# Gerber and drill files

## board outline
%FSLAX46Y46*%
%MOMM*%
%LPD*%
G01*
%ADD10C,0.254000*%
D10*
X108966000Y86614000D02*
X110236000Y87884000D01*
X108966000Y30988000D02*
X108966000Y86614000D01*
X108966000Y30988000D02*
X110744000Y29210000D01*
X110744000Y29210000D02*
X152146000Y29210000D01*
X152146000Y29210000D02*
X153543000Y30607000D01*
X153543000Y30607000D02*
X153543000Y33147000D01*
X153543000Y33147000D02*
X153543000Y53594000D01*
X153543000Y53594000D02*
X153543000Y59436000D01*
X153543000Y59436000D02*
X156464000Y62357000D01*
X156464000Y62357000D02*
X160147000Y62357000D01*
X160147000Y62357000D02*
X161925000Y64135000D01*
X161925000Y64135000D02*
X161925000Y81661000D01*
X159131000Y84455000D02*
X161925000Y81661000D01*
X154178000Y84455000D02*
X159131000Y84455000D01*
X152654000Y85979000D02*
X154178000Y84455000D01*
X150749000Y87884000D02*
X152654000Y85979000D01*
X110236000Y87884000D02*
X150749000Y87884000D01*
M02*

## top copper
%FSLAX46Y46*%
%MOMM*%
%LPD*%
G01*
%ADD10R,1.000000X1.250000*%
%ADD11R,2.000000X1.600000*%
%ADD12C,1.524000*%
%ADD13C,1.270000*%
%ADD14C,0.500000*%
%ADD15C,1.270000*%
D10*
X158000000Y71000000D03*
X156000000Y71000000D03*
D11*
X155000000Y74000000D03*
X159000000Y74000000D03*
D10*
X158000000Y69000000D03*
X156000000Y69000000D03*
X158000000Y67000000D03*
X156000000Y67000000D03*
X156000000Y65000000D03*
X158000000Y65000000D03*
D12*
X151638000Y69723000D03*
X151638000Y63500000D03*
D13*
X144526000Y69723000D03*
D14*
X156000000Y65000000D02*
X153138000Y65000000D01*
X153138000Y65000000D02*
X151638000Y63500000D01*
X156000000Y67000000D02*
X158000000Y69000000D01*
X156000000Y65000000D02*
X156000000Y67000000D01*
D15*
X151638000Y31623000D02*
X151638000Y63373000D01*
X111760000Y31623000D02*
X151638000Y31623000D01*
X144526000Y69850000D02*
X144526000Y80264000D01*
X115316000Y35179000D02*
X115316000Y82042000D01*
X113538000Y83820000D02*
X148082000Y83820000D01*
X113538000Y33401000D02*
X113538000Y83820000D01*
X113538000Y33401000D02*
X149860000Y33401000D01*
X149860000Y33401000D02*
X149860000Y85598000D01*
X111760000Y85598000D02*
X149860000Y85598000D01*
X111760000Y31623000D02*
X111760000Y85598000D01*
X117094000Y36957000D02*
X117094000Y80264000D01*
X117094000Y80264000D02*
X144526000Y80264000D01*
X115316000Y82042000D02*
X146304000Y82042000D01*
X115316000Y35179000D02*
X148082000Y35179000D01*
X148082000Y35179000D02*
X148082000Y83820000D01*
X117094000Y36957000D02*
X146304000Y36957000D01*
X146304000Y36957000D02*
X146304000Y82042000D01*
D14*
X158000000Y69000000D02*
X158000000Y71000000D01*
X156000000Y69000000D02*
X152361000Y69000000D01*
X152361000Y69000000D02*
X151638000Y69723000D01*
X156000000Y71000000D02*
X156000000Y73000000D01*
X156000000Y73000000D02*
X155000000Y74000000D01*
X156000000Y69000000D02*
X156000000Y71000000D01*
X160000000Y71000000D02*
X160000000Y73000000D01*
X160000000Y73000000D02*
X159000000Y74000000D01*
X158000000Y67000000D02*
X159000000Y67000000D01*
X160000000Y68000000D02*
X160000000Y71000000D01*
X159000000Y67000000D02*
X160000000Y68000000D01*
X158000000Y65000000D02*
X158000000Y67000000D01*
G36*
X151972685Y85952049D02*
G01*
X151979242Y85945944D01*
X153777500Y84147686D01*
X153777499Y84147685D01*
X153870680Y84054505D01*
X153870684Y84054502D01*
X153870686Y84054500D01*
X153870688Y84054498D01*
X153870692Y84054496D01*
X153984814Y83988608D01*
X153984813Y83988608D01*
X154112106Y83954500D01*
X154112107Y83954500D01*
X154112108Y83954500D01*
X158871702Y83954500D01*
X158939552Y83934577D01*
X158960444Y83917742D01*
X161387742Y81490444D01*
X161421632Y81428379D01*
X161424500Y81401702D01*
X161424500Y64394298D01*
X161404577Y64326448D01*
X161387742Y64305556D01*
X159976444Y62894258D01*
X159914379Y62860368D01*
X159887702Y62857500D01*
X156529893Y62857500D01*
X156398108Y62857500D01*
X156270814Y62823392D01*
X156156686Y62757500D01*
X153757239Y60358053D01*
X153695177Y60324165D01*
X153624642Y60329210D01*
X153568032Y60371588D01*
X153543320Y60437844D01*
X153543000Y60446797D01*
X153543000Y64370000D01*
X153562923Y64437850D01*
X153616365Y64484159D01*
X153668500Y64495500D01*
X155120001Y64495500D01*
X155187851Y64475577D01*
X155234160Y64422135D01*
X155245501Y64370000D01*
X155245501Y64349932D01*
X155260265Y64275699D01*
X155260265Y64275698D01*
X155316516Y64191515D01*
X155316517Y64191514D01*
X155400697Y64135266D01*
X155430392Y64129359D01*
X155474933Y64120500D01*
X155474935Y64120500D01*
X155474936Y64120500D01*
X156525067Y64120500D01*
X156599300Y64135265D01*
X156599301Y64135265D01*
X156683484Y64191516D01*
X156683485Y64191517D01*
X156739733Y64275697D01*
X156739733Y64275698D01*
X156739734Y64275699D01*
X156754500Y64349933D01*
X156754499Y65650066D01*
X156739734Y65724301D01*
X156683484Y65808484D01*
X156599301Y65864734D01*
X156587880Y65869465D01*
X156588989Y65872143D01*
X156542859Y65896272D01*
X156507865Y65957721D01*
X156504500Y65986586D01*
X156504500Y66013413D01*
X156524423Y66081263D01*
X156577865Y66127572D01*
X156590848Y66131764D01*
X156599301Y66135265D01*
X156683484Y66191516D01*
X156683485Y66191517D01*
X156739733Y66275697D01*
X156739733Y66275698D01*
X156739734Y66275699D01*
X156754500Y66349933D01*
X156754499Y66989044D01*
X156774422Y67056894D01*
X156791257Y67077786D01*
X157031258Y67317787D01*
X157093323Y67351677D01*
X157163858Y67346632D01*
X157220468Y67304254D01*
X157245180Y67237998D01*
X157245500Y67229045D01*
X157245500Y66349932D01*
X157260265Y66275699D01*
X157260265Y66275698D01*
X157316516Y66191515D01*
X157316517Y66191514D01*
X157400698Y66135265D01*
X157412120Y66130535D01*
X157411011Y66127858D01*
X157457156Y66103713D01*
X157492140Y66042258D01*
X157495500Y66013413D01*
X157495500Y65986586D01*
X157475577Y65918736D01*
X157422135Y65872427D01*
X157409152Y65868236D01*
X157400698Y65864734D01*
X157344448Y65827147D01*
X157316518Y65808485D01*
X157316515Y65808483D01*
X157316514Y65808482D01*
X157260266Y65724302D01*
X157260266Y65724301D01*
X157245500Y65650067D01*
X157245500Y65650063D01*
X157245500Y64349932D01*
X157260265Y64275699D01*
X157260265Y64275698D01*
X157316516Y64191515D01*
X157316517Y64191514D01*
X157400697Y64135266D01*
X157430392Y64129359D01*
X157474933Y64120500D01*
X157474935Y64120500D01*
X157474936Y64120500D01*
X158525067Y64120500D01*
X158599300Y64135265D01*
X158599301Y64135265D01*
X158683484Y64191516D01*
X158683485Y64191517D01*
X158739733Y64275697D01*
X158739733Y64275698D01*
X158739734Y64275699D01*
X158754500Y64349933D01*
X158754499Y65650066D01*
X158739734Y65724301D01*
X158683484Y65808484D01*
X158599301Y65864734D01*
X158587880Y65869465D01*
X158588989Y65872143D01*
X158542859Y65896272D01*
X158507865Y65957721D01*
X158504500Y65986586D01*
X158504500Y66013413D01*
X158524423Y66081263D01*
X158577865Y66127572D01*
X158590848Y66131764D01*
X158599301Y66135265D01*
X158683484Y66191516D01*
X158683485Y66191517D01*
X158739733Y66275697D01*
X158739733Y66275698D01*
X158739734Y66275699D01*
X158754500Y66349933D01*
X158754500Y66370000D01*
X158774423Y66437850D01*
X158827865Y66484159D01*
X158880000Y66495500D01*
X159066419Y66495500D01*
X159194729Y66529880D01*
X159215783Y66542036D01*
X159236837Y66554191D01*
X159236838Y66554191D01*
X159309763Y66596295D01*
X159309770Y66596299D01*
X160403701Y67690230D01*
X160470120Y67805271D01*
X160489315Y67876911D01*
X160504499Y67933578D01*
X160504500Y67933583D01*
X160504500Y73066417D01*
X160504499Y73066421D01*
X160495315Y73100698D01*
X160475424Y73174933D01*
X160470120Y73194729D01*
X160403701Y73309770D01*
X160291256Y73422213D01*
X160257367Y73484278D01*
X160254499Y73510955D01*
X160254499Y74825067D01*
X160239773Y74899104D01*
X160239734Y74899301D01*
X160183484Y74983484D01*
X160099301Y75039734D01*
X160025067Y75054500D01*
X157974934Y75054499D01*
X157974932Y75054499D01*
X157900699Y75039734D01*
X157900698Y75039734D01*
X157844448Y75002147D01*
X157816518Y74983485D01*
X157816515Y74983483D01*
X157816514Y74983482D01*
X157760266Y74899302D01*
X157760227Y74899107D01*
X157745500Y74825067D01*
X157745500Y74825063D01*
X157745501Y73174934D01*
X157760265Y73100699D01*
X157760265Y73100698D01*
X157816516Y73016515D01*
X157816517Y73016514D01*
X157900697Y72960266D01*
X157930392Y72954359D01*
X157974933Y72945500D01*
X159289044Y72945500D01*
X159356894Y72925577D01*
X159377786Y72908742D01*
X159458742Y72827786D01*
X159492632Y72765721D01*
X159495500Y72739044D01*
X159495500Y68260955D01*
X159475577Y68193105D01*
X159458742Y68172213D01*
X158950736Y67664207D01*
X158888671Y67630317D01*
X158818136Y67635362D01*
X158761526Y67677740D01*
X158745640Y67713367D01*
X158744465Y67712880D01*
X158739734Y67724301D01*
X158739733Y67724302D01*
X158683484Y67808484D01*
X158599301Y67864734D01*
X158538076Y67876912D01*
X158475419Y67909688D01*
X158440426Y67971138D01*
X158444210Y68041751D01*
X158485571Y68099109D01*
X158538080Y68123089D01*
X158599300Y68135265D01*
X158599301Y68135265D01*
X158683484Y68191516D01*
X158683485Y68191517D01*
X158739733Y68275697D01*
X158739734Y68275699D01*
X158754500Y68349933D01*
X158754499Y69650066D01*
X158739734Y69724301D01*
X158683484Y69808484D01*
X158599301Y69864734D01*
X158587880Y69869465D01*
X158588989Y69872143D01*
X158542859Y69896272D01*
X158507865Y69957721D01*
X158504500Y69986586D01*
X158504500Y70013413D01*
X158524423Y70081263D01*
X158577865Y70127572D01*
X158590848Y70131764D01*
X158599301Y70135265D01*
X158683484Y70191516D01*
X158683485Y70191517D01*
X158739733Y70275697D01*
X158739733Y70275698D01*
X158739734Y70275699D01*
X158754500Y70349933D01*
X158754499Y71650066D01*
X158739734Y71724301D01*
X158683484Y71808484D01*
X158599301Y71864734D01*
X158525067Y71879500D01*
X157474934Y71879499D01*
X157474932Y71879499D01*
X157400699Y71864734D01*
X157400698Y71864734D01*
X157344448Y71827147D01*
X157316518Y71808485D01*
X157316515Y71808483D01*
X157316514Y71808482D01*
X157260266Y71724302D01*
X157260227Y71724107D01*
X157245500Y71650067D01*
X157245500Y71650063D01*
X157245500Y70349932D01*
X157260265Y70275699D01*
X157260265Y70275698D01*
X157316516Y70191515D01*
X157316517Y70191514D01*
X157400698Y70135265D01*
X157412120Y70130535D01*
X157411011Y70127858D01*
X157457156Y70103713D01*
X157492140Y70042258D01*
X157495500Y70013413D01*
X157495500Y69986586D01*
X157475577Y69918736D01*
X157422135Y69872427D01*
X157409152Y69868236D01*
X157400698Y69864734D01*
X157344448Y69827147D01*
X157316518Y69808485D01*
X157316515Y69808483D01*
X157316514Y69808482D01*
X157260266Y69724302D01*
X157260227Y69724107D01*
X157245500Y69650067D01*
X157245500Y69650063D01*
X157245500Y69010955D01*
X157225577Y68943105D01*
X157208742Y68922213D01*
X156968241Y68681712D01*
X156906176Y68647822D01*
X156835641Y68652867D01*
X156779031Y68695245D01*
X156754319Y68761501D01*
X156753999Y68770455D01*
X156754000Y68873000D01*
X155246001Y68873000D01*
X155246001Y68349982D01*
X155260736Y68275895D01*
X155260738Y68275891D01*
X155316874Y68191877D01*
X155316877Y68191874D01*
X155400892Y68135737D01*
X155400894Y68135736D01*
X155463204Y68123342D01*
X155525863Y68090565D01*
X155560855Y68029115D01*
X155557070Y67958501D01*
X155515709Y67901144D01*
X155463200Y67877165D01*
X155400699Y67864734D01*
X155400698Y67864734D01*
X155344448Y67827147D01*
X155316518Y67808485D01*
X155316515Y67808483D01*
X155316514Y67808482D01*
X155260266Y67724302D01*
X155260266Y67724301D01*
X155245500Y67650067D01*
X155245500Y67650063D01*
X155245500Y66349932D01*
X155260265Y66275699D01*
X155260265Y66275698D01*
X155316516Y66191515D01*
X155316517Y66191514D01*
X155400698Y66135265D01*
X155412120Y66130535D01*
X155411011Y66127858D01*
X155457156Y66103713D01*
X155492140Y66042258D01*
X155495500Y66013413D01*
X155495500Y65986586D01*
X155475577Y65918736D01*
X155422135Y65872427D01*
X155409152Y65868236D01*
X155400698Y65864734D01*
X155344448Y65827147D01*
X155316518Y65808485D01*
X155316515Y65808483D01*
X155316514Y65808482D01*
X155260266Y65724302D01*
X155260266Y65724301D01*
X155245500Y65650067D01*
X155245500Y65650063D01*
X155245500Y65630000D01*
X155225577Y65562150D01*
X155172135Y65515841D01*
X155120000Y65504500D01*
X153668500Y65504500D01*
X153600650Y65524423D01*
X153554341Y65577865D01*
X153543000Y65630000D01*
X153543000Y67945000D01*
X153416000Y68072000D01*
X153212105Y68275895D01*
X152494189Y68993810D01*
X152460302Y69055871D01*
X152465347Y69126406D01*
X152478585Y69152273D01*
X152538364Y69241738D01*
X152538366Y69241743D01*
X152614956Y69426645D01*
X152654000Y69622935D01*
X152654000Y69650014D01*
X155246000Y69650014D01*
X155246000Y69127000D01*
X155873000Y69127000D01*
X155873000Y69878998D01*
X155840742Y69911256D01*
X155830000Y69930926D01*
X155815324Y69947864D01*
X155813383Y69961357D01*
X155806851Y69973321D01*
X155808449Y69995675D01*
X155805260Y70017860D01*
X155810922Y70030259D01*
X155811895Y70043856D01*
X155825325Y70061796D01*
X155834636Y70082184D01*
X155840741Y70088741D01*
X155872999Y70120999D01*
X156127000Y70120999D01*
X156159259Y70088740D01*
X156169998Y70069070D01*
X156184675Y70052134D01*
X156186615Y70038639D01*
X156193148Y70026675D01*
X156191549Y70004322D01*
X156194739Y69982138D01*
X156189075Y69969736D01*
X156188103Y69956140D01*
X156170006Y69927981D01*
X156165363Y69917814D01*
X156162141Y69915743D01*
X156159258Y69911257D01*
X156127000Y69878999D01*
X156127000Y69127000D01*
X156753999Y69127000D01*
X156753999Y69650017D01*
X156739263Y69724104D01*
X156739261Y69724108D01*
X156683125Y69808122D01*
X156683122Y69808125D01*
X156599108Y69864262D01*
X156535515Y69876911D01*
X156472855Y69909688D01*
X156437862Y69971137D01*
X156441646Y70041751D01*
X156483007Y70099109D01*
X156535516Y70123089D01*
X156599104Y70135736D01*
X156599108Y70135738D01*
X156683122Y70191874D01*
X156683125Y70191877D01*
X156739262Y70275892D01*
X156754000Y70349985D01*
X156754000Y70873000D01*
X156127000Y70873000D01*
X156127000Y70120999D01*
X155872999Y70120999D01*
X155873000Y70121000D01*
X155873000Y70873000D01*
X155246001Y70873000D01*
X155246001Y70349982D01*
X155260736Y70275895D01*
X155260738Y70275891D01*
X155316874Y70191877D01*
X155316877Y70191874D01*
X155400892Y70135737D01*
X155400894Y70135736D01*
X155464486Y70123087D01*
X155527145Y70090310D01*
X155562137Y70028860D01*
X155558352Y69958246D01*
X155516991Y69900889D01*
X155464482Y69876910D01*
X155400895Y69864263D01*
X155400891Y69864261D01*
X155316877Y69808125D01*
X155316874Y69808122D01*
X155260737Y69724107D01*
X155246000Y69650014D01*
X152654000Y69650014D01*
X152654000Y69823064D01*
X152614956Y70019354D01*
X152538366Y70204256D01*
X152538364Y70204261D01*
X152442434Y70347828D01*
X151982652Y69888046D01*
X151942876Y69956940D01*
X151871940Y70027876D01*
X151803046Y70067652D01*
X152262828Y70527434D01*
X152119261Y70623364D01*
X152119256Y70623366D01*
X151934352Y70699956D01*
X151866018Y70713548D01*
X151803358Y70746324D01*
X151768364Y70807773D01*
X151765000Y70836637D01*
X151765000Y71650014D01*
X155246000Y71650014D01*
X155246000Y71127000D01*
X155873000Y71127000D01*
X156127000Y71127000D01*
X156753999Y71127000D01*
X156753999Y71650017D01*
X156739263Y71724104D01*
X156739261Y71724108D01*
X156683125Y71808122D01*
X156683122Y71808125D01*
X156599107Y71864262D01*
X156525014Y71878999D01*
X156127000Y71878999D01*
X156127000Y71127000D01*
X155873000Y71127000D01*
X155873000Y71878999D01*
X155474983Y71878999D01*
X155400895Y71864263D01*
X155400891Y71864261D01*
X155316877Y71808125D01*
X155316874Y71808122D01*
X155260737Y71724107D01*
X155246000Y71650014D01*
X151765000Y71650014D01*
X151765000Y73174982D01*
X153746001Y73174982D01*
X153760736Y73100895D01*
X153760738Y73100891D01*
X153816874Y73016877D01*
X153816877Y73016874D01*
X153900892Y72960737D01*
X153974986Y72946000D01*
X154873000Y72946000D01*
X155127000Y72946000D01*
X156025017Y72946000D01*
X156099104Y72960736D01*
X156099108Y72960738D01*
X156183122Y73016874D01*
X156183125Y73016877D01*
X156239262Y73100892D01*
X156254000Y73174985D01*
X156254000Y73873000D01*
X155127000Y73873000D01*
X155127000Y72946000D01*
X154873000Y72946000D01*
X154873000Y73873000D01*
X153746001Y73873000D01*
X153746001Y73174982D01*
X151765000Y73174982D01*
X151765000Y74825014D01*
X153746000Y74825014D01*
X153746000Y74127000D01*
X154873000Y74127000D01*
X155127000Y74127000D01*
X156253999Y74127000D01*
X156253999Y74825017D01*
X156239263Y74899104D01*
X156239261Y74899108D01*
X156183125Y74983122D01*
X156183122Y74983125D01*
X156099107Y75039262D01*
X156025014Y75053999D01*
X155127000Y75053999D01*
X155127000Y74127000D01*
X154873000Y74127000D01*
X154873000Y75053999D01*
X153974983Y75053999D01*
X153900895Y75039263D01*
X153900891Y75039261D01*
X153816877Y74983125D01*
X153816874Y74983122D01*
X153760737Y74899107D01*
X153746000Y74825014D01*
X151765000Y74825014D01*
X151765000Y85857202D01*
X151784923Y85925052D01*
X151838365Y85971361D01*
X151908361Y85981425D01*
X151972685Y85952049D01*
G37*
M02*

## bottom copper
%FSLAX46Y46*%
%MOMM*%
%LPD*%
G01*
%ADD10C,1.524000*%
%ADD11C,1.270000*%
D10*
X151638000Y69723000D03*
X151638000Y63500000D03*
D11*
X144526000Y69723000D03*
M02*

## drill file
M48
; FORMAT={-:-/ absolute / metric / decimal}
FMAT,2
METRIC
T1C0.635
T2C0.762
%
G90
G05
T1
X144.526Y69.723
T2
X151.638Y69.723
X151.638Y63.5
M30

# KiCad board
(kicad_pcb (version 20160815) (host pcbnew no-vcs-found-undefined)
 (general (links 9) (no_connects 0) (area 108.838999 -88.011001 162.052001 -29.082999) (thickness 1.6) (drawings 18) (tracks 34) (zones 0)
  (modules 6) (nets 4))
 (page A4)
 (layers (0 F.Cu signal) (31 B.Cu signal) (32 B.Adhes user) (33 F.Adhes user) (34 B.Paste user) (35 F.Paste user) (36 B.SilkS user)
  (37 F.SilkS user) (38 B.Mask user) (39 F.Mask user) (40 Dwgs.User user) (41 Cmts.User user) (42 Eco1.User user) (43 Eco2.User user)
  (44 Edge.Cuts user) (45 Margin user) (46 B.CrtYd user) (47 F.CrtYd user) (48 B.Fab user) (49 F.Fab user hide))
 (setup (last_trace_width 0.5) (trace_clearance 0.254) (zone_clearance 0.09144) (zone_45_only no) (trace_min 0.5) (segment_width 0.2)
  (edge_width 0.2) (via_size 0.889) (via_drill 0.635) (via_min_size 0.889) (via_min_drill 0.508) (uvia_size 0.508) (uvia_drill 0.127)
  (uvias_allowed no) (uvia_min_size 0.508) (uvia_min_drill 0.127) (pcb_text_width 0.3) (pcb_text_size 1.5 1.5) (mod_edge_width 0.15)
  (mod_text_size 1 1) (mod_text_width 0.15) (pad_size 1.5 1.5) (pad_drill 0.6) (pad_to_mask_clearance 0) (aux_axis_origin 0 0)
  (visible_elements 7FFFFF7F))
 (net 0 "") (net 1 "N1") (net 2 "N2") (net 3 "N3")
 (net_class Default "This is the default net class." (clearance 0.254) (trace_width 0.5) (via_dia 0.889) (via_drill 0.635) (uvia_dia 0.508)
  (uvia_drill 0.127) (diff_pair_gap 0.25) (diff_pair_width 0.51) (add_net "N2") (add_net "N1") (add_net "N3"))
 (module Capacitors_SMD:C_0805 (layer F.Cu) (at 157 -71)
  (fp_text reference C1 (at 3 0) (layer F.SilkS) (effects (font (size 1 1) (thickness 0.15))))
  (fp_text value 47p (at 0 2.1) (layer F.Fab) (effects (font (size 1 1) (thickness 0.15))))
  (pad 2 smd rect (at 1 0) (size 1 1.25) (layers F.Cu F.Paste F.Mask) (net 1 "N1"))
  (pad 1 smd rect (at -1 0) (size 1 1.25) (layers F.Cu F.Paste F.Mask) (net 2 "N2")))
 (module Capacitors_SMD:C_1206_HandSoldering (layer F.Cu) (at 157 -74 180)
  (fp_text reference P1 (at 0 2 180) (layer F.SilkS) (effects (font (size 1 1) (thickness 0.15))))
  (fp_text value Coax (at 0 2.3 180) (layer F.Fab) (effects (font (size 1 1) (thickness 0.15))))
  (pad 2 smd rect (at 2 0 180) (size 2 1.6) (layers F.Cu F.Paste F.Mask) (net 2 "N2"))
  (pad 1 smd rect (at -2 0 180) (size 2 1.6) (layers F.Cu F.Paste F.Mask) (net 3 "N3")))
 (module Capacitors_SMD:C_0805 (layer F.Cu) (at 157 -69)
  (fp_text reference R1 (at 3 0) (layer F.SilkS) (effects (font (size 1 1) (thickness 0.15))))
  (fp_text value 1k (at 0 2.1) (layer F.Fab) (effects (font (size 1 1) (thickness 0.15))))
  (pad 2 smd rect (at 1 0) (size 1 1.25) (layers F.Cu F.Paste F.Mask) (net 1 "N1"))
  (pad 1 smd rect (at -1 0) (size 1 1.25) (layers F.Cu F.Paste F.Mask) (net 2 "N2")))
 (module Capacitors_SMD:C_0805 (layer F.Cu) (at 157 -67)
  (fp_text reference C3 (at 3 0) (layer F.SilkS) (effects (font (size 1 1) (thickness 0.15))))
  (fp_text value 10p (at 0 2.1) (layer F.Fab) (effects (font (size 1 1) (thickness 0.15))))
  (pad 2 smd rect (at 1 0) (size 1 1.25) (layers F.Cu F.Paste F.Mask) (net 3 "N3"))
  (pad 1 smd rect (at -1 0) (size 1 1.25) (layers F.Cu F.Paste F.Mask) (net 1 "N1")))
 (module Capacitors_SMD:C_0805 (layer F.Cu) (at 157 -65)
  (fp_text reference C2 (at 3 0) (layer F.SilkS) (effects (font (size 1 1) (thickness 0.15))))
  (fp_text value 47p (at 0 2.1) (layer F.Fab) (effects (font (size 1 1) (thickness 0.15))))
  (pad 1 smd rect (at -1 0) (size 1 1.25) (layers F.Cu F.Paste F.Mask) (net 1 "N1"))
  (pad 2 smd rect (at 1 0) (size 1 1.25) (layers F.Cu F.Paste F.Mask) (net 3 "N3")))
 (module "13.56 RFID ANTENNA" (layer F.Cu) (at 111.76 -31.623)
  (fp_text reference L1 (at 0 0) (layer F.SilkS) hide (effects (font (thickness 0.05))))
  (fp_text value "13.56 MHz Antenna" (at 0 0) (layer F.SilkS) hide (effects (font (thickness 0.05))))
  (pad 2 thru_hole circle (at 39.878 -38.1) (size 1.524 1.524) (drill 0.762) (layers *.Cu *.Paste *.Mask) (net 2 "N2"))
  (pad 1 thru_hole circle (at 39.878 -31.877) (size 1.524 1.524) (drill 0.762) (layers *.Cu *.Paste *.Mask) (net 1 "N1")))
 (gr_line (start 108.966 -86.614) (end 110.236 -87.884) (layer Edge.Cuts) (width 0.254))
 (gr_line (start 108.966 -30.988) (end 108.966 -86.614) (layer Edge.Cuts) (width 0.254))
 (gr_line (start 108.966 -30.988) (end 110.744 -29.21) (layer Edge.Cuts) (width 0.254))
 (gr_line (start 110.744 -29.21) (end 152.146 -29.21) (layer Edge.Cuts) (width 0.254))
 (gr_line (start 152.146 -29.21) (end 153.543 -30.607) (layer Edge.Cuts) (width 0.254))
 (gr_line (start 153.543 -30.607) (end 153.543 -33.147) (layer Edge.Cuts) (width 0.254))
 (gr_line (start 153.543 -33.147) (end 153.543 -53.594) (layer Edge.Cuts) (width 0.254))
 (gr_line (start 153.543 -53.594) (end 153.543 -59.436) (layer Edge.Cuts) (width 0.254))
 (gr_line (start 153.543 -59.436) (end 156.464 -62.357) (layer Edge.Cuts) (width 0.254))
 (gr_line (start 156.464 -62.357) (end 160.147 -62.357) (layer Edge.Cuts) (width 0.254))
 (gr_line (start 160.147 -62.357) (end 161.925 -64.135) (layer Edge.Cuts) (width 0.254))
 (gr_line (start 161.925 -64.135) (end 161.925 -81.661) (layer Edge.Cuts) (width 0.254))
 (gr_line (start 159.131 -84.455) (end 161.925 -81.661) (layer Edge.Cuts) (width 0.254))
 (gr_line (start 154.178 -84.455) (end 159.131 -84.455) (layer Edge.Cuts) (width 0.254))
 (gr_line (start 152.654 -85.979) (end 154.178 -84.455) (layer Edge.Cuts) (width 0.254))
 (gr_line (start 150.749 -87.884) (end 152.654 -85.979) (layer Edge.Cuts) (width 0.254))
 (gr_line (start 110.236 -87.884) (end 150.749 -87.884) (layer Edge.Cuts) (width 0.254))
 (segment (start 156 -65) (end 153.138 -65) (width 0.5) (layer F.Cu) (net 1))
 (segment (start 153.138 -65) (end 151.638 -63.5) (width 0.5) (layer F.Cu) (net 1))
 (segment (start 156 -67) (end 158 -69) (width 0.5) (layer F.Cu) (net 1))
 (segment (start 156 -65) (end 156 -67) (width 0.5) (layer F.Cu) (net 1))
 (via (at 144.526 -69.723) (size 1.27) (layers F.Cu B.Cu) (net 1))
 (segment (start 151.638 -31.623) (end 151.638 -63.373) (width 1.27) (layer F.Cu) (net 1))
 (segment (start 111.76 -31.623) (end 151.638 -31.623) (width 1.27) (layer F.Cu) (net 1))
 (segment (start 144.526 -69.85) (end 144.526 -80.264) (width 1.27) (layer F.Cu) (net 1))
 (segment (start 115.316 -35.179) (end 115.316 -82.042) (width 1.27) (layer F.Cu) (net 1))
 (segment (start 113.538 -83.82) (end 148.082 -83.82) (width 1.27) (layer F.Cu) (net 1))
 (segment (start 113.538 -33.401) (end 113.538 -83.82) (width 1.27) (layer F.Cu) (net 1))
 (segment (start 113.538 -33.401) (end 149.86 -33.401) (width 1.27) (layer F.Cu) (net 1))
 (segment (start 149.86 -33.401) (end 149.86 -85.598) (width 1.27) (layer F.Cu) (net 1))
 (segment (start 111.76 -85.598) (end 149.86 -85.598) (width 1.27) (layer F.Cu) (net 1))
 (segment (start 111.76 -31.623) (end 111.76 -85.598) (width 1.27) (layer F.Cu) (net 1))
 (segment (start 117.094 -36.957) (end 117.094 -80.264) (width 1.27) (layer F.Cu) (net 1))
 (segment (start 117.094 -80.264) (end 144.526 -80.264) (width 1.27) (layer F.Cu) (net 1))
 (segment (start 115.316 -82.042) (end 146.304 -82.042) (width 1.27) (layer F.Cu) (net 1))
 (segment (start 115.316 -35.179) (end 148.082 -35.179) (width 1.27) (layer F.Cu) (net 1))
 (segment (start 148.082 -35.179) (end 148.082 -83.82) (width 1.27) (layer F.Cu) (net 1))
 (segment (start 117.094 -36.957) (end 146.304 -36.957) (width 1.27) (layer F.Cu) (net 1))
 (segment (start 146.304 -36.957) (end 146.304 -82.042) (width 1.27) (layer F.Cu) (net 1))
 (segment (start 158 -69) (end 158 -71) (width 0.5) (layer F.Cu) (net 1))
 (segment (start 156 -69) (end 152.361 -69) (width 0.5) (layer F.Cu) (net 2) (status 400000))
 (segment (start 152.361 -69) (end 151.638 -69.723) (width 0.5) (layer F.Cu) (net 2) (status 800000))
 (segment (start 156 -71) (end 156 -73) (width 0.5) (layer F.Cu) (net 2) (status 400000))
 (segment (start 156 -73) (end 155 -74) (width 0.5) (layer F.Cu) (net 2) (status 800000))
 (segment (start 156 -69) (end 156 -71) (width 0.5) (layer F.Cu) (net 2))
 (segment (start 160 -71) (end 160 -73) (width 0.5) (layer F.Cu) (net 3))
 (segment (start 160 -73) (end 159 -74) (width 0.5) (layer F.Cu) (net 3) (status 800000))
 (segment (start 158 -67) (end 159 -67) (width 0.5) (layer F.Cu) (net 3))
 (segment (start 160 -68) (end 160 -71) (width 0.5) (layer F.Cu) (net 3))
 (segment (start 159 -67) (end 160 -68) (width 0.5) (layer F.Cu) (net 3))
 (segment (start 158 -65) (end 158 -67) (width 0.5) (layer F.Cu) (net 3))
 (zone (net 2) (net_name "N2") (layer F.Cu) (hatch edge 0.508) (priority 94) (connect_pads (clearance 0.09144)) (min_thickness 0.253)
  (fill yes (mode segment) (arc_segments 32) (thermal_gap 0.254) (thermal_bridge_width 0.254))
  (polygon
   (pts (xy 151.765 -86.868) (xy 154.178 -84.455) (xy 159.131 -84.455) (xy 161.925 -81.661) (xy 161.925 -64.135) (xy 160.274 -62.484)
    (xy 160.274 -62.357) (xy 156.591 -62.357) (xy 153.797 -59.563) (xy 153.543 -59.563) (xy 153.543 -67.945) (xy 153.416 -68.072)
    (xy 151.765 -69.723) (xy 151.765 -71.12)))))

